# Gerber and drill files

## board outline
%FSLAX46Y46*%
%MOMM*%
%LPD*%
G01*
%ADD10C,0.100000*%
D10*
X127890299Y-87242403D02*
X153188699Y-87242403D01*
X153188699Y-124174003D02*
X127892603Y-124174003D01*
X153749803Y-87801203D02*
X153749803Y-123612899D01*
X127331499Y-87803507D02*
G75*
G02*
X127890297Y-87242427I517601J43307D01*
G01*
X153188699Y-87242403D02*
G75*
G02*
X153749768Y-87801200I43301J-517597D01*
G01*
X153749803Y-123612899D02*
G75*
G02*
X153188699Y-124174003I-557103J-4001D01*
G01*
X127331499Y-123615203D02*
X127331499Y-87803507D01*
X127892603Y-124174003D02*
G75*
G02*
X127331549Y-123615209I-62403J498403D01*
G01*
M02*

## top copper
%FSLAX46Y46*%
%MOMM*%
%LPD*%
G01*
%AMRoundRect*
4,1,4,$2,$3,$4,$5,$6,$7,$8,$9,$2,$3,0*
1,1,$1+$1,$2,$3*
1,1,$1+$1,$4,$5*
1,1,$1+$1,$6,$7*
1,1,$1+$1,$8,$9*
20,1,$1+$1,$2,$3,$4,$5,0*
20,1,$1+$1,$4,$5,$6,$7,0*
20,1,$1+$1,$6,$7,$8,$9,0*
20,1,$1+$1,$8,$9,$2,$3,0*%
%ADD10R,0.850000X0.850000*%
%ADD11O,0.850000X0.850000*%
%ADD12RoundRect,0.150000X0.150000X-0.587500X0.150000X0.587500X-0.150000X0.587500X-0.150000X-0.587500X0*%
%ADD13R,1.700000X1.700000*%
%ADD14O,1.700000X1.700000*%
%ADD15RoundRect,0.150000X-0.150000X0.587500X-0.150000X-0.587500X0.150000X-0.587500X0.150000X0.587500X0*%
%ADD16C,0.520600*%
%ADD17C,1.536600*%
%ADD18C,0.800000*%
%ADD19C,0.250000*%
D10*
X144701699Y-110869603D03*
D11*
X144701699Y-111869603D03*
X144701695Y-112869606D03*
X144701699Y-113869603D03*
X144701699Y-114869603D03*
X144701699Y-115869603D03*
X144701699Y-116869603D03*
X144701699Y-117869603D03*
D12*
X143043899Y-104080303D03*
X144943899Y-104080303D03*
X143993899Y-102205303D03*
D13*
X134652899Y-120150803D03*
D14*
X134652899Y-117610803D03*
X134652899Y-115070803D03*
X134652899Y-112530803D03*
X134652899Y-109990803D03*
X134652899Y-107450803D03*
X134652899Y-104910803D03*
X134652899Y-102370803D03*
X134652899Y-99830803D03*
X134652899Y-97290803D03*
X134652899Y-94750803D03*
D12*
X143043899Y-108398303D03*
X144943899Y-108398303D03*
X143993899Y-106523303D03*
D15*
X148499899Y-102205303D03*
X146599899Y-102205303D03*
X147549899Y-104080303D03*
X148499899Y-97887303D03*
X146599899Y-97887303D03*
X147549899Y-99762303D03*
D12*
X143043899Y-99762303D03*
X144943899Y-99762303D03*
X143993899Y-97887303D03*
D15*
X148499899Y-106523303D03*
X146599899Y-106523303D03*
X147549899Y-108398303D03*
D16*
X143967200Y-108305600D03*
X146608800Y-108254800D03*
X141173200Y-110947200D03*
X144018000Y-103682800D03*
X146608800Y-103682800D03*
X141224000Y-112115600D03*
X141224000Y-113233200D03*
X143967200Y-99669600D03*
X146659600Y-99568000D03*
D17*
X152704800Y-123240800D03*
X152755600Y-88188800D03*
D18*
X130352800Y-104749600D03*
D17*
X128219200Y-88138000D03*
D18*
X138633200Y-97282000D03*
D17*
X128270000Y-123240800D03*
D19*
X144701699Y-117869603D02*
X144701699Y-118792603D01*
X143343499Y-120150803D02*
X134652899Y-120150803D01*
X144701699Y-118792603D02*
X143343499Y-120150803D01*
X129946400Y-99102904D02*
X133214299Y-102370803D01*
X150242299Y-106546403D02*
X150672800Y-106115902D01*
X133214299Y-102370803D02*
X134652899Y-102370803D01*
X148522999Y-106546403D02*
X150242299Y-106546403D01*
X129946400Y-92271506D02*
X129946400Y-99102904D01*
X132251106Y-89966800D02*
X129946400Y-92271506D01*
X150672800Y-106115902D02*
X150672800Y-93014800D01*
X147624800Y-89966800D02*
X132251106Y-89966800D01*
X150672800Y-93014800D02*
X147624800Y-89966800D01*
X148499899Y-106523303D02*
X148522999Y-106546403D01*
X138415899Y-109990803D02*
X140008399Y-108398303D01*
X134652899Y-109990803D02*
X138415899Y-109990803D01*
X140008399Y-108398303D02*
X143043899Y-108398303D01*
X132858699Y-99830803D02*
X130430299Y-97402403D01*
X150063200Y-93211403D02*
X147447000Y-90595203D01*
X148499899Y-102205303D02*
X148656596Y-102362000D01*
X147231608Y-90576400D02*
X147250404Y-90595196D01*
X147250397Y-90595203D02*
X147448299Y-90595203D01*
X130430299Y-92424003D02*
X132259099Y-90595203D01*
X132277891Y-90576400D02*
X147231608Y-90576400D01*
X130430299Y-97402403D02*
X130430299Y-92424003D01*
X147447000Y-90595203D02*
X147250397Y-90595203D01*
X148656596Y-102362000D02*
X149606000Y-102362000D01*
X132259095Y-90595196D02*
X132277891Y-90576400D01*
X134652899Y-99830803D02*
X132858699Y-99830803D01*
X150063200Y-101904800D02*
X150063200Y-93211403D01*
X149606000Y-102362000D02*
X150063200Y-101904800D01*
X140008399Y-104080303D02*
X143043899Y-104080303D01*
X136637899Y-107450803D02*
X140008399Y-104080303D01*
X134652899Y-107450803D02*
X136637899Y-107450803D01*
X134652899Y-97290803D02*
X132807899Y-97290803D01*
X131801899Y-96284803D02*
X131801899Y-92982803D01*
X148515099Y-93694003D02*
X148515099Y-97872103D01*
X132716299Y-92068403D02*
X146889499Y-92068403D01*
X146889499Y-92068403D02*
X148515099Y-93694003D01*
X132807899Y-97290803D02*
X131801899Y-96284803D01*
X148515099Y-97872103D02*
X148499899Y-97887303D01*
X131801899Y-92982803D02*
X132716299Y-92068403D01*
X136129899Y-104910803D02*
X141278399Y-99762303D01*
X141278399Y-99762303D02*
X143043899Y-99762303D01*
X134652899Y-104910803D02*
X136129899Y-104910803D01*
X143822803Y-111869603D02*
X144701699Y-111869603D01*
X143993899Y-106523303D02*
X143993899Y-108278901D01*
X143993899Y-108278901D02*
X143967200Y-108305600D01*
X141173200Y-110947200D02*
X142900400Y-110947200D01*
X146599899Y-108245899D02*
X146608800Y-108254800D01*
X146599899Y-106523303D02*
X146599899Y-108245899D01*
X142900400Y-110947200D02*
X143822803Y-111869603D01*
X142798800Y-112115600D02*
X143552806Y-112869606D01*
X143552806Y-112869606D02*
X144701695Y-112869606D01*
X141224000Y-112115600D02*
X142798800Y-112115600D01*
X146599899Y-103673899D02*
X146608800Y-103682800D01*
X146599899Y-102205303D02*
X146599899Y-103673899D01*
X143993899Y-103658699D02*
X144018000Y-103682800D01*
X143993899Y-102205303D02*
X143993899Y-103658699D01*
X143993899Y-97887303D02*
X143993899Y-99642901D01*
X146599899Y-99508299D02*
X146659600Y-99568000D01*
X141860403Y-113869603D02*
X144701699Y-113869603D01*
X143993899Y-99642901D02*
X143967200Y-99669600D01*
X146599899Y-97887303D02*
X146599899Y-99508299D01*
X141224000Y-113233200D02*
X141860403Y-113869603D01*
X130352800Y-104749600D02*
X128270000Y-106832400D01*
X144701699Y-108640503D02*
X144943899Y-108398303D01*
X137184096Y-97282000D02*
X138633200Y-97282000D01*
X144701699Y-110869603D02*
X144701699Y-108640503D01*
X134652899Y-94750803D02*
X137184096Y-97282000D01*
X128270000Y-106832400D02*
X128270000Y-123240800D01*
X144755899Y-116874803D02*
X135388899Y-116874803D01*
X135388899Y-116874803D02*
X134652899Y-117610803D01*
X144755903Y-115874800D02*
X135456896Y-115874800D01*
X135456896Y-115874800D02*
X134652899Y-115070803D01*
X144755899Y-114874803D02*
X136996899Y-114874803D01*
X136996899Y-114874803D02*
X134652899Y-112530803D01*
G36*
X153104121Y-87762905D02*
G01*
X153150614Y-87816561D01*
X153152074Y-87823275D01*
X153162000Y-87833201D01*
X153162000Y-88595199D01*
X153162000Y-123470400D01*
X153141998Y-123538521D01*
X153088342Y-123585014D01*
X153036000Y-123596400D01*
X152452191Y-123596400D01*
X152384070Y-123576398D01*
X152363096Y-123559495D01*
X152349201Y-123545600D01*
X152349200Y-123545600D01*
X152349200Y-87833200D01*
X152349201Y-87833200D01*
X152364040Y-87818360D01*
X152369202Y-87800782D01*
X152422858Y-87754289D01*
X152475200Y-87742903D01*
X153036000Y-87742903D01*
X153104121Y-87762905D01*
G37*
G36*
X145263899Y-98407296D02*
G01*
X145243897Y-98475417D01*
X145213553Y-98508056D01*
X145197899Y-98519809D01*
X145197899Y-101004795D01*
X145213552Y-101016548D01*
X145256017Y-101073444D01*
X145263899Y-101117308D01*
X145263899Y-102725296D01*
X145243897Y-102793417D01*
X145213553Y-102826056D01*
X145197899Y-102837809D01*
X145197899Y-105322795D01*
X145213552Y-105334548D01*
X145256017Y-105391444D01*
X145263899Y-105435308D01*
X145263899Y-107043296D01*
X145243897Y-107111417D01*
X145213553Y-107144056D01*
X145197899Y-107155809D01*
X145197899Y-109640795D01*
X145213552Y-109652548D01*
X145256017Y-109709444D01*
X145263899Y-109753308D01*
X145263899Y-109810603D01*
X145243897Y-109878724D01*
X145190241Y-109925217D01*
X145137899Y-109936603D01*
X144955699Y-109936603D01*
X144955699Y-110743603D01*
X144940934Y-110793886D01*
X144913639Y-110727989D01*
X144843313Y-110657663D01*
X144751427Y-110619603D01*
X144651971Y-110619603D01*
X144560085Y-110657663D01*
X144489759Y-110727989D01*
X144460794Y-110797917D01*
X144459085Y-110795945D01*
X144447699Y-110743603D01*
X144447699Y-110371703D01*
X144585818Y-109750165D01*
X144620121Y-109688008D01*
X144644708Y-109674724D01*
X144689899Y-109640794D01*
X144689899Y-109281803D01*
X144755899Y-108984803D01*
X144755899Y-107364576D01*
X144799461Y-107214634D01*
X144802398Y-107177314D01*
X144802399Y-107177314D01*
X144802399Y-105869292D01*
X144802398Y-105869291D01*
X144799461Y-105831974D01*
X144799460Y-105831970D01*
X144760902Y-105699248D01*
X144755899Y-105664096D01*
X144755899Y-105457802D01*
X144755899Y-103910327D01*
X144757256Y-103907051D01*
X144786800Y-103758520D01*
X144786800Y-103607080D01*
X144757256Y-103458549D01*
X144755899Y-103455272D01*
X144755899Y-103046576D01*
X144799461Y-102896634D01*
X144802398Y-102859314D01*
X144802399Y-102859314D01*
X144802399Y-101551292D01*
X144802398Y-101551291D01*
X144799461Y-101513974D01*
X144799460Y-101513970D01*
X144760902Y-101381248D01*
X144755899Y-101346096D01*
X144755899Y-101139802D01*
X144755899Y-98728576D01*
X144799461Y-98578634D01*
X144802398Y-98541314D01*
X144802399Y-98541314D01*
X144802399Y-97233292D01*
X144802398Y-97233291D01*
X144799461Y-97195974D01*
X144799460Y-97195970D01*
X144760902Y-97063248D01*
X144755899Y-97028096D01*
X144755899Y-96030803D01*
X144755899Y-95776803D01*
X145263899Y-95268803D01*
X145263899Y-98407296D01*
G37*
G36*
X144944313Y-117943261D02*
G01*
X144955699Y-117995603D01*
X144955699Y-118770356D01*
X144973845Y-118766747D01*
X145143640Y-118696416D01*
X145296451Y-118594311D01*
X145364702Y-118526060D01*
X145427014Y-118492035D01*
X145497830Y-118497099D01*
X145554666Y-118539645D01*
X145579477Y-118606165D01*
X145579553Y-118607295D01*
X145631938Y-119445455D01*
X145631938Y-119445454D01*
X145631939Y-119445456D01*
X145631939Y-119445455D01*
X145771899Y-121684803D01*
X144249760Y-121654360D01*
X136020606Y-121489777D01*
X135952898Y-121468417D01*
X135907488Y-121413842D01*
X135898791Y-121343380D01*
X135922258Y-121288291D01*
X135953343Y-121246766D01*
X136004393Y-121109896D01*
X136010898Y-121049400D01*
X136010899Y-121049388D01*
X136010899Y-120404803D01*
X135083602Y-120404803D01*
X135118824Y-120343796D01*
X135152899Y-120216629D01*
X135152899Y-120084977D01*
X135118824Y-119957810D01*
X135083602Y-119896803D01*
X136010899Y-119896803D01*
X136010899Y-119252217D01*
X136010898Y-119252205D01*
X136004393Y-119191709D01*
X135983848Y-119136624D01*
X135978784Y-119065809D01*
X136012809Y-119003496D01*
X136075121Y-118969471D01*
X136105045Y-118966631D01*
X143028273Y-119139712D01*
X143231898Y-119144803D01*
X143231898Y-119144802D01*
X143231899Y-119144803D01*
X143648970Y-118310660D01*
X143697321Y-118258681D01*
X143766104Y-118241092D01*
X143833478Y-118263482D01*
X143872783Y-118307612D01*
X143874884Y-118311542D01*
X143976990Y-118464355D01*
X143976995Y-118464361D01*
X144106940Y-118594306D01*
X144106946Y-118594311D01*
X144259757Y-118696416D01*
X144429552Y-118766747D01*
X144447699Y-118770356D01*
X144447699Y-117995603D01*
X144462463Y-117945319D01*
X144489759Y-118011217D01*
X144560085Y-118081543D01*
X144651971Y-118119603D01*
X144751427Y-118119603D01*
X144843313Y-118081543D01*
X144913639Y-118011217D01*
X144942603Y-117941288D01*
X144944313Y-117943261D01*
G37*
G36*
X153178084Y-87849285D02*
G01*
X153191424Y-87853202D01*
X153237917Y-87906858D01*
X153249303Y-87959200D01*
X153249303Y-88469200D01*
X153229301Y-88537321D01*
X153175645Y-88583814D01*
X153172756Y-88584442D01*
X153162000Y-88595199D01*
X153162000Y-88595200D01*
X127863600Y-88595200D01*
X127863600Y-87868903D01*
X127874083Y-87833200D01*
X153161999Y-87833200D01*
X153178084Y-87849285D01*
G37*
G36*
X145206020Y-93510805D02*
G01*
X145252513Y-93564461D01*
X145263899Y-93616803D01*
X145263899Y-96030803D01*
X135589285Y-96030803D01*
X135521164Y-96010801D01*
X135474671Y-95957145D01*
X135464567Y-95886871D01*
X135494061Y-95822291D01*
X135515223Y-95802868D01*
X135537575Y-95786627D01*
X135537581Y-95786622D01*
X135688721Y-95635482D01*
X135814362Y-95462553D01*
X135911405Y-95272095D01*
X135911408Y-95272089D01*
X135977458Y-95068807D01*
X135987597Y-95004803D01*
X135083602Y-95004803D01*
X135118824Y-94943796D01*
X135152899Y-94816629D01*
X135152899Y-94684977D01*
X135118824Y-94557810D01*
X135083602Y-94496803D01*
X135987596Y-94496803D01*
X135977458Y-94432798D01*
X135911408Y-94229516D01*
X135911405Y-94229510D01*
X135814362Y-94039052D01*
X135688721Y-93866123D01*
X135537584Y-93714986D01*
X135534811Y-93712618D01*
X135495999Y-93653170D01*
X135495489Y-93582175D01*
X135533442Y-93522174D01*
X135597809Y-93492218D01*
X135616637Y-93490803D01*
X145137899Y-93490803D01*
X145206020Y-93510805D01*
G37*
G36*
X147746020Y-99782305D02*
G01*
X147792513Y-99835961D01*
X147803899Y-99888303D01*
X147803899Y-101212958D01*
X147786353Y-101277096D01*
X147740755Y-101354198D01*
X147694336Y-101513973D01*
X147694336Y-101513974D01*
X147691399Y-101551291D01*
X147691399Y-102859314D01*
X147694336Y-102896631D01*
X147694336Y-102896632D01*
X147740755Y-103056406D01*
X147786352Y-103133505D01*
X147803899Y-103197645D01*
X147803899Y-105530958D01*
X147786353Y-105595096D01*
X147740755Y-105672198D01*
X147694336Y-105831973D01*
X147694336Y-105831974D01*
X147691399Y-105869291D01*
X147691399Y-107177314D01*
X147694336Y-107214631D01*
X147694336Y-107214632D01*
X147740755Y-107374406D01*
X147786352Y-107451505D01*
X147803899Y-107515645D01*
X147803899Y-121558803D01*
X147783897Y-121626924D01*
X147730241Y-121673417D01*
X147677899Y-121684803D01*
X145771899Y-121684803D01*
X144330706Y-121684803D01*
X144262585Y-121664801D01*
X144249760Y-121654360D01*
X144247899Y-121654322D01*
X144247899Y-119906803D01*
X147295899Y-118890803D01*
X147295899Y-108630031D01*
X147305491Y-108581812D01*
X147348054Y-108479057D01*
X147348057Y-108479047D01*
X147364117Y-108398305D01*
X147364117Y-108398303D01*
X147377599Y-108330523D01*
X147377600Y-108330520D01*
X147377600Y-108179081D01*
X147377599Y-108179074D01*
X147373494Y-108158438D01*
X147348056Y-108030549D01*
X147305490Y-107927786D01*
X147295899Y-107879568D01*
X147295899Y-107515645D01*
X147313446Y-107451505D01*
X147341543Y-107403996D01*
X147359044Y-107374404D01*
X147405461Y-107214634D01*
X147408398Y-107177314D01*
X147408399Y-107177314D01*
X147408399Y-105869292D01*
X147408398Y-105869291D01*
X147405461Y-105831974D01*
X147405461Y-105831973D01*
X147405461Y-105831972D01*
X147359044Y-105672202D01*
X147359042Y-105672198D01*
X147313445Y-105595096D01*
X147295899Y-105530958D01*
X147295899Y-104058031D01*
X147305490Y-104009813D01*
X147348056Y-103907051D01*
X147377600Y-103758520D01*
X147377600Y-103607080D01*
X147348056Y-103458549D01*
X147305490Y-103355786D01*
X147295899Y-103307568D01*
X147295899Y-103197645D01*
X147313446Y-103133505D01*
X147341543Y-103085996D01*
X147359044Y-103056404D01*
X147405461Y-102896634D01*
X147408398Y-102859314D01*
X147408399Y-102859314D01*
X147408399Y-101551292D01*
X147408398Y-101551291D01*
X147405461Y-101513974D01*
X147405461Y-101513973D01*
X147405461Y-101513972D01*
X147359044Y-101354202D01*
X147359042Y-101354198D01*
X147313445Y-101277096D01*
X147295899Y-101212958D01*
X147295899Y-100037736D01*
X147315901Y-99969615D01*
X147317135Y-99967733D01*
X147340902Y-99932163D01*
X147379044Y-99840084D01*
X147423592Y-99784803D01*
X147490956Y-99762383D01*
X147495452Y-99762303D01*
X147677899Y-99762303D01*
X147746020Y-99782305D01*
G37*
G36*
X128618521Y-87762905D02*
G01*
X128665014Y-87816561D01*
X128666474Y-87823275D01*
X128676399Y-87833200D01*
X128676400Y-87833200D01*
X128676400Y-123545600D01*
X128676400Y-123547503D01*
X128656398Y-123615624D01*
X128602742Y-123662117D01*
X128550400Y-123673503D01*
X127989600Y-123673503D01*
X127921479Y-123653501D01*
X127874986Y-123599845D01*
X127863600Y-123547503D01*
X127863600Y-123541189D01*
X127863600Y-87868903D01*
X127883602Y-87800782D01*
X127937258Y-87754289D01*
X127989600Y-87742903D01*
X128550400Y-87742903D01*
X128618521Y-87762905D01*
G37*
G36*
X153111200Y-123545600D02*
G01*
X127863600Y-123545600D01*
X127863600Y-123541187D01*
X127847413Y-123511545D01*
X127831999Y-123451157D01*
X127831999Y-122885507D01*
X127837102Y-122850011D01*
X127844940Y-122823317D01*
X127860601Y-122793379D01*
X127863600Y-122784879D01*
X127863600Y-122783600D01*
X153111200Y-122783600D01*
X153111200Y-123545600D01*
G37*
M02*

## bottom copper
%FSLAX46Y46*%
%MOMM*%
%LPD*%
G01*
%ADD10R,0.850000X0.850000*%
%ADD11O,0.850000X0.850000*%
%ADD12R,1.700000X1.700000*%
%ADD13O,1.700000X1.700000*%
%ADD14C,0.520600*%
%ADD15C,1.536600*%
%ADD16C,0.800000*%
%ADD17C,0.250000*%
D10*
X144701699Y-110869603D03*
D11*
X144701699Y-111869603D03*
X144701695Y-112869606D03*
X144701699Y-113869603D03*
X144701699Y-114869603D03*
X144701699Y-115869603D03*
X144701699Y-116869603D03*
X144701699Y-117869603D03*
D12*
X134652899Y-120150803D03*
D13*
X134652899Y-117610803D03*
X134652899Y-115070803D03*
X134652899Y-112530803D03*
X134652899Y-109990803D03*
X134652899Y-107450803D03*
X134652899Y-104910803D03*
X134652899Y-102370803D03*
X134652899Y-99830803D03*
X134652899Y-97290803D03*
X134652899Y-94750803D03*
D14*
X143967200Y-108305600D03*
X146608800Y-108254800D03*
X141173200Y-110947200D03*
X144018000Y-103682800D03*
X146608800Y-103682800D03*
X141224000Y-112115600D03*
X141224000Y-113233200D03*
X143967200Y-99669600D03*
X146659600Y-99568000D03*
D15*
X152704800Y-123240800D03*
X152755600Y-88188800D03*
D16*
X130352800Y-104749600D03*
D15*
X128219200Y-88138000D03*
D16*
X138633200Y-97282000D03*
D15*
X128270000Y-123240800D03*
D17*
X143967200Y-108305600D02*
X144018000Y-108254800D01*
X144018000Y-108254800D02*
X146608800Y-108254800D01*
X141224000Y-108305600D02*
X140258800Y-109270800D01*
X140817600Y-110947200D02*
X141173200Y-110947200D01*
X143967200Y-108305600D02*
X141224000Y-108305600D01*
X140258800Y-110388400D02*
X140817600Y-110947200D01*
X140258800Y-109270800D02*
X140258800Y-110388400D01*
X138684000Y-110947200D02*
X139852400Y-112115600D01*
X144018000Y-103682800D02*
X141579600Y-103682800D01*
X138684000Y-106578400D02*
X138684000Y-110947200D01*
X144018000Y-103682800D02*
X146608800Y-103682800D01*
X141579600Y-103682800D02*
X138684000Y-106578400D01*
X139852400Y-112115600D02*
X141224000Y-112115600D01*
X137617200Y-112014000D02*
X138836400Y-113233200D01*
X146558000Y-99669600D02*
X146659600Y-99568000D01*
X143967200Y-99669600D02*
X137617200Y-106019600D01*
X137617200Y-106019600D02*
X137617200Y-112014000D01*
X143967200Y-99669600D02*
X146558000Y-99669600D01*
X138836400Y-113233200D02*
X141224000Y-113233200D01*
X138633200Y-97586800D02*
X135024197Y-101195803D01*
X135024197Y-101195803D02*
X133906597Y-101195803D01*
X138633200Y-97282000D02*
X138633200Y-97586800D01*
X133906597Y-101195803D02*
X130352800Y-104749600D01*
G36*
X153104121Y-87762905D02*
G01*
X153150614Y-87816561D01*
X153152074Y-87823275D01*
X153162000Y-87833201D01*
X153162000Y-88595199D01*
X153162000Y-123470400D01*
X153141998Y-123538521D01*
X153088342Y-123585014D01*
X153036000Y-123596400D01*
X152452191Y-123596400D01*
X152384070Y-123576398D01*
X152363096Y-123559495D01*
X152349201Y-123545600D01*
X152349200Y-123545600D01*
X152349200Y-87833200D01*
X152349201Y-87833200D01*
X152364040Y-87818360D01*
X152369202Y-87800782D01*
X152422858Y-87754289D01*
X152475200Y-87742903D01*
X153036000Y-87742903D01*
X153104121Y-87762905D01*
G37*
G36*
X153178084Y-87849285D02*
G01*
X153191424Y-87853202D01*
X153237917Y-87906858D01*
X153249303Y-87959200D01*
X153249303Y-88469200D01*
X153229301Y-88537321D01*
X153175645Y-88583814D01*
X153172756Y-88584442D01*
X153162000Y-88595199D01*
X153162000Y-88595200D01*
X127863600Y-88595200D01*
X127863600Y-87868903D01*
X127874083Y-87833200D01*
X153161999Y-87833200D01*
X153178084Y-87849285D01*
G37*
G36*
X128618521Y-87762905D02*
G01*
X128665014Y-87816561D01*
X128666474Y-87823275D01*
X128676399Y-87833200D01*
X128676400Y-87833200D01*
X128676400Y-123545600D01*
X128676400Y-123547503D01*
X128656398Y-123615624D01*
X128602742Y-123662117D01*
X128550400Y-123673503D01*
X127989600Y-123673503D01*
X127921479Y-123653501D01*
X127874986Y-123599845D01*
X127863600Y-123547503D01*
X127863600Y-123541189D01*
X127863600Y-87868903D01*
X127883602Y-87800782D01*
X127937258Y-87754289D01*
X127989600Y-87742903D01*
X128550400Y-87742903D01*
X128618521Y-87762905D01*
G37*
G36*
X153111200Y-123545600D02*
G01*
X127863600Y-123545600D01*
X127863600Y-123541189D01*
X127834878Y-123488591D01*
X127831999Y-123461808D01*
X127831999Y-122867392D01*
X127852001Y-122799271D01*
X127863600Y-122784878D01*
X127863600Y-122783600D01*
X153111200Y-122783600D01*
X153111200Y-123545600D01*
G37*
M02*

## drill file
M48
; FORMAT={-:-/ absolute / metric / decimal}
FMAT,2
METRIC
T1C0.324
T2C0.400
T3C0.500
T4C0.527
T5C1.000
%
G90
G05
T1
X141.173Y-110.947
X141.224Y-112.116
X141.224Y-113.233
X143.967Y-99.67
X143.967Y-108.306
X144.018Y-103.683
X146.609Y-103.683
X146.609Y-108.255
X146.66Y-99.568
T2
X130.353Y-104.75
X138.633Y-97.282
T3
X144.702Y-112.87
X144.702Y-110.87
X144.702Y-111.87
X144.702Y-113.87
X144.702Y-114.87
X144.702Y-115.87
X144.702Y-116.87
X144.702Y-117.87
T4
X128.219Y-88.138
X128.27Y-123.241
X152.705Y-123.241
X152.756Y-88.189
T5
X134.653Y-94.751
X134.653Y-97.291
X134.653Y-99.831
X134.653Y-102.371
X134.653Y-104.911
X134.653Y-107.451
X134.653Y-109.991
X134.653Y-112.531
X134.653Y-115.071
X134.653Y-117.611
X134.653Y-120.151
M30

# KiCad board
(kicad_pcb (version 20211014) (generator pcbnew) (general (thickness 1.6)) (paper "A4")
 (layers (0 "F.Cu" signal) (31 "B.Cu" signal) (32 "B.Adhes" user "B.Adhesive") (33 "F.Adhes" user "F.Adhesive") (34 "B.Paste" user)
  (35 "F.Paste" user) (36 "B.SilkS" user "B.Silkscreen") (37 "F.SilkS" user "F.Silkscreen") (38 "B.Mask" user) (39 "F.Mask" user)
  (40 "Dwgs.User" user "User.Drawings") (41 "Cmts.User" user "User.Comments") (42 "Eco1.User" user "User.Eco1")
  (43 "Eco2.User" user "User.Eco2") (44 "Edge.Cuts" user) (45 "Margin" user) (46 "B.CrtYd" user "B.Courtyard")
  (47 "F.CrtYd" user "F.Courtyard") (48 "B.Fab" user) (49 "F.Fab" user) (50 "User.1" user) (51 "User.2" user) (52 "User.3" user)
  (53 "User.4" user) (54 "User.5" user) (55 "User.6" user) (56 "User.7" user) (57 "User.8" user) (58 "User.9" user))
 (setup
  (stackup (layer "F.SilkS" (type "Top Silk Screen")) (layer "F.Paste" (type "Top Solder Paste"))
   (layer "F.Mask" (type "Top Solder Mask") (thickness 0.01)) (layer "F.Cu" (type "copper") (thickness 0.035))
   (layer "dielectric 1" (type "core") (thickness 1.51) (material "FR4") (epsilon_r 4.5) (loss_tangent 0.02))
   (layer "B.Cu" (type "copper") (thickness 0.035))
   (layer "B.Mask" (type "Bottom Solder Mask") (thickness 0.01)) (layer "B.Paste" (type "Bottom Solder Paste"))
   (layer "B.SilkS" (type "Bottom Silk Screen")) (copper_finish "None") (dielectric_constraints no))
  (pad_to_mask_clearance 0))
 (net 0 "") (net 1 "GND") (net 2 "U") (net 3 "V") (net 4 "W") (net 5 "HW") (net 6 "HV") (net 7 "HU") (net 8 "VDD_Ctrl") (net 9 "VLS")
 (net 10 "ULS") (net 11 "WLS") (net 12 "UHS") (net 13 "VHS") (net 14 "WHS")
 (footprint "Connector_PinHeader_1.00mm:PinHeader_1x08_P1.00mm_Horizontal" (layer "F.Cu") (at 144.701699 110.869603)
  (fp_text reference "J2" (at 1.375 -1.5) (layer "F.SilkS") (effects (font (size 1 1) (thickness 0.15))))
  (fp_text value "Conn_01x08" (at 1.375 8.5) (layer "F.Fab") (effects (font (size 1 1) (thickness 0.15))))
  (pad "1" thru_hole rect (at 0 0) (size 0.85 0.85) (drill 0.5) (layers *.Cu *.Mask) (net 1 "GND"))
  (pad "2" thru_hole oval (at 0 1) (size 0.85 0.85) (drill 0.5) (layers *.Cu *.Mask) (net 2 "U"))
  (pad "3" thru_hole oval (at -0.000004 2.000003) (size 0.85 0.85) (drill 0.5) (layers *.Cu *.Mask) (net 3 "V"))
  (pad "4" thru_hole oval (at 0 3) (size 0.85 0.85) (drill 0.5) (layers *.Cu *.Mask) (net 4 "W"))
  (pad "5" thru_hole oval (at 0 4) (size 0.85 0.85) (drill 0.5) (layers *.Cu *.Mask) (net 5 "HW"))
  (pad "6" thru_hole oval (at 0 5) (size 0.85 0.85) (drill 0.5) (layers *.Cu *.Mask) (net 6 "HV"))
  (pad "7" thru_hole oval (at 0 6) (size 0.85 0.85) (drill 0.5) (layers *.Cu *.Mask) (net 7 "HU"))
  (pad "8" thru_hole oval (at 0 7) (size 0.85 0.85) (drill 0.5) (layers *.Cu *.Mask) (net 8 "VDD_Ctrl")))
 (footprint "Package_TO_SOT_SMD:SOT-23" (layer "F.Cu") (at 143.993899 103.142803 90)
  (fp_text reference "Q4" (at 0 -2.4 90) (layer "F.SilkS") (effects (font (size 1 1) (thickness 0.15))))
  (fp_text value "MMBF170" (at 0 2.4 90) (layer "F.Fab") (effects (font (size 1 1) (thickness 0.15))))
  (pad "1" smd roundrect (at -0.9375 -0.95 90) (size 1.475 0.6) (layers "F.Cu" "F.Paste" "F.Mask") (roundrect_rratio 0.25) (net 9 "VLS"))
  (pad "2" smd roundrect (at -0.9375 0.95 90) (size 1.475 0.6) (layers "F.Cu" "F.Paste" "F.Mask") (roundrect_rratio 0.25) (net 1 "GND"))
  (pad "3" smd roundrect (at 0.9375 0 90) (size 1.475 0.6) (layers "F.Cu" "F.Paste" "F.Mask") (roundrect_rratio 0.25) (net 3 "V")))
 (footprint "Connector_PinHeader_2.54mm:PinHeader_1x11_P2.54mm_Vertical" (layer "F.Cu") (at 134.652899 120.150803 180)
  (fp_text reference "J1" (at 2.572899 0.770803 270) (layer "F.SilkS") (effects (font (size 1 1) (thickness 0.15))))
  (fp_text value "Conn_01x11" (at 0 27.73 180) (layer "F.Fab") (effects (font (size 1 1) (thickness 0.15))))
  (pad "1" thru_hole rect (at 0 0 180) (size 1.7 1.7) (drill 1) (layers *.Cu *.Mask) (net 8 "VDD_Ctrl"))
  (pad "2" thru_hole oval (at 0 2.54 180) (size 1.7 1.7) (drill 1) (layers *.Cu *.Mask) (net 7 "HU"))
  (pad "3" thru_hole oval (at 0 5.08 180) (size 1.7 1.7) (drill 1) (layers *.Cu *.Mask) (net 6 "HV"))
  (pad "4" thru_hole oval (at 0 7.62 180) (size 1.7 1.7) (drill 1) (layers *.Cu *.Mask) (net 5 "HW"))
  (pad "5" thru_hole oval (at 0 10.16 180) (size 1.7 1.7) (drill 1) (layers *.Cu *.Mask) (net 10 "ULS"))
  (pad "6" thru_hole oval (at 0 12.7 180) (size 1.7 1.7) (drill 1) (layers *.Cu *.Mask) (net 9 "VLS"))
  (pad "7" thru_hole oval (at 0 15.24 180) (size 1.7 1.7) (drill 1) (layers *.Cu *.Mask) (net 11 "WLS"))
  (pad "8" thru_hole oval (at 0 17.78 180) (size 1.7 1.7) (drill 1) (layers *.Cu *.Mask) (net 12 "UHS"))
  (pad "9" thru_hole oval (at 0 20.32 180) (size 1.7 1.7) (drill 1) (layers *.Cu *.Mask) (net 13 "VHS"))
  (pad "10" thru_hole oval (at 0 22.86 180) (size 1.7 1.7) (drill 1) (layers *.Cu *.Mask) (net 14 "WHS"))
  (pad "11" thru_hole oval (at 0 25.4 180) (size 1.7 1.7) (drill 1) (layers *.Cu *.Mask) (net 1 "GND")))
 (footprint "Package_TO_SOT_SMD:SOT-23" (layer "F.Cu") (at 143.993899 107.460803 90)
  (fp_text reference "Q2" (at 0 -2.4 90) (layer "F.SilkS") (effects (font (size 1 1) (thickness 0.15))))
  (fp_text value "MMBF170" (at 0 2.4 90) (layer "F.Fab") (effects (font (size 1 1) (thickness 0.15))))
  (pad "1" smd roundrect (at -0.9375 -0.95 90) (size 1.475 0.6) (layers "F.Cu" "F.Paste" "F.Mask") (roundrect_rratio 0.25) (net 10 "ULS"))
  (pad "2" smd roundrect (at -0.9375 0.95 90) (size 1.475 0.6) (layers "F.Cu" "F.Paste" "F.Mask") (roundrect_rratio 0.25) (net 1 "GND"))
  (pad "3" smd roundrect (at 0.9375 0 90) (size 1.475 0.6) (layers "F.Cu" "F.Paste" "F.Mask") (roundrect_rratio 0.25) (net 2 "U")))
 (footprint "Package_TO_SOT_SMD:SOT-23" (layer "F.Cu") (at 147.549899 103.142803 -90)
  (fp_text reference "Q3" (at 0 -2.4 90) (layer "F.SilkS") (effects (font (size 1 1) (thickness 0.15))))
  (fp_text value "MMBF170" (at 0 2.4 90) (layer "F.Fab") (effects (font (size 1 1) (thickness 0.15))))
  (pad "1" smd roundrect (at -0.9375 -0.95 270) (size 1.475 0.6) (layers "F.Cu" "F.Paste" "F.Mask") (roundrect_rratio 0.25) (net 13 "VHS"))
  (pad "2" smd roundrect (at -0.9375 0.95 270) (size 1.475 0.6) (layers "F.Cu" "F.Paste" "F.Mask") (roundrect_rratio 0.25) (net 3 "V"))
  (pad "3" smd roundrect (at 0.9375 0 270) (size 1.475 0.6) (layers "F.Cu" "F.Paste" "F.Mask") (roundrect_rratio 0.25) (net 8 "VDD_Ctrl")))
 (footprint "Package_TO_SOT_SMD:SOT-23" (layer "F.Cu") (at 147.549899 98.824803 -90)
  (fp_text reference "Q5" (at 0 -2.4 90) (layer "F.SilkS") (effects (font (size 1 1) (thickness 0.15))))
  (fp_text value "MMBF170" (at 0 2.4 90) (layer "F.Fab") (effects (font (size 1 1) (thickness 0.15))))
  (pad "1" smd roundrect (at -0.9375 -0.95 270) (size 1.475 0.6) (layers "F.Cu" "F.Paste" "F.Mask") (roundrect_rratio 0.25) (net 14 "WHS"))
  (pad "2" smd roundrect (at -0.9375 0.95 270) (size 1.475 0.6) (layers "F.Cu" "F.Paste" "F.Mask") (roundrect_rratio 0.25) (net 4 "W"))
  (pad "3" smd roundrect (at 0.9375 0 270) (size 1.475 0.6) (layers "F.Cu" "F.Paste" "F.Mask") (roundrect_rratio 0.25) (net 8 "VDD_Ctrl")))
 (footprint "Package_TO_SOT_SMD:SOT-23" (layer "F.Cu") (at 143.993899 98.824803 90)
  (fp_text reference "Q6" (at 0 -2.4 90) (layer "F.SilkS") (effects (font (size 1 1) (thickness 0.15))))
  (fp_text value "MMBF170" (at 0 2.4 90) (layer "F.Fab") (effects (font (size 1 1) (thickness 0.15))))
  (pad "1" smd roundrect (at -0.9375 -0.95 90) (size 1.475 0.6) (layers "F.Cu" "F.Paste" "F.Mask") (roundrect_rratio 0.25) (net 11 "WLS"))
  (pad "2" smd roundrect (at -0.9375 0.95 90) (size 1.475 0.6) (layers "F.Cu" "F.Paste" "F.Mask") (roundrect_rratio 0.25) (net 1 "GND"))
  (pad "3" smd roundrect (at 0.9375 0 90) (size 1.475 0.6) (layers "F.Cu" "F.Paste" "F.Mask") (roundrect_rratio 0.25) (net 4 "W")))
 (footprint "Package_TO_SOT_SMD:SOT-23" (layer "F.Cu") (at 147.549899 107.460803 -90)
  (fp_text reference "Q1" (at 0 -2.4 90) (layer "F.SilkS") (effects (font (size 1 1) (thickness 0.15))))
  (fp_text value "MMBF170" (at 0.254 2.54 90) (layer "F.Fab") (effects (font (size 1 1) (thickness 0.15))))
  (pad "1" smd roundrect (at -0.9375 -0.95 270) (size 1.475 0.6) (layers "F.Cu" "F.Paste" "F.Mask") (roundrect_rratio 0.25) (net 12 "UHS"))
  (pad "2" smd roundrect (at -0.9375 0.95 270) (size 1.475 0.6) (layers "F.Cu" "F.Paste" "F.Mask") (roundrect_rratio 0.25) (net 2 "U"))
  (pad "3" smd roundrect (at 0.9375 0 270) (size 1.475 0.6) (layers "F.Cu" "F.Paste" "F.Mask") (roundrect_rratio 0.25) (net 8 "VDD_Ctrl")))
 (gr_line (start 127.890299 87.242403) (end 153.188699 87.242403) (layer "Edge.Cuts") (width 0.1))
 (gr_line (start 153.188699 124.174003) (end 127.892603 124.174003) (layer "Edge.Cuts") (width 0.1))
 (gr_line (start 153.749803 87.801203) (end 153.749803 123.612899) (layer "Edge.Cuts") (width 0.1))
 (gr_arc (start 127.331499 87.803507) (mid 127.481074 87.393663) (end 127.890299 87.242403) (layer "Edge.Cuts") (width 0.1))
 (gr_arc (start 153.188699 87.242403) (mid 153.598538 87.391982) (end 153.749803 87.801203) (layer "Edge.Cuts") (width 0.1))
 (gr_arc (start 153.749803 123.612899) (mid 153.586636 124.010836) (end 153.188699 124.174003) (layer "Edge.Cuts") (width 0.1))
 (gr_line (start 127.331499 123.615203) (end 127.331499 87.803507) (layer "Edge.Cuts") (width 0.1))
 (gr_arc (start 127.892603 124.174003) (mid 127.475721 124.031493) (end 127.331499 123.615203) (layer "Edge.Cuts") (width 0.1))
 (segment (start 144.701699 117.869603) (end 144.701699 118.792603) (width 0.25) (layer "F.Cu") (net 8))
 (segment (start 143.343499 120.150803) (end 134.652899 120.150803) (width 0.25) (layer "F.Cu") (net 8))
 (segment (start 144.701699 118.792603) (end 143.343499 120.150803) (width 0.25) (layer "F.Cu") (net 8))
 (segment (start 129.9464 99.102904) (end 133.214299 102.370803) (width 0.25) (layer "F.Cu") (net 12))
 (segment (start 150.242299 106.546403) (end 150.6728 106.115902) (width 0.25) (layer "F.Cu") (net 12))
 (segment (start 133.214299 102.370803) (end 134.652899 102.370803) (width 0.25) (layer "F.Cu") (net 12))
 (segment (start 148.522999 106.546403) (end 150.242299 106.546403) (width 0.25) (layer "F.Cu") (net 12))
 (segment (start 129.9464 92.271506) (end 129.9464 99.102904) (width 0.25) (layer "F.Cu") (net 12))
 (segment (start 132.251106 89.9668) (end 129.9464 92.271506) (width 0.25) (layer "F.Cu") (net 12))
 (segment (start 150.6728 106.115902) (end 150.6728 93.0148) (width 0.25) (layer "F.Cu") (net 12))
 (segment (start 147.6248 89.9668) (end 132.251106 89.9668) (width 0.25) (layer "F.Cu") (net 12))
 (segment (start 150.6728 93.0148) (end 147.6248 89.9668) (width 0.25) (layer "F.Cu") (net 12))
 (segment (start 148.499899 106.523303) (end 148.522999 106.546403) (width 0.25) (layer "F.Cu") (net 12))
 (segment (start 138.415899 109.990803) (end 140.008399 108.398303) (width 0.25) (layer "F.Cu") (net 10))
 (segment (start 134.652899 109.990803) (end 138.415899 109.990803) (width 0.25) (layer "F.Cu") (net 10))
 (segment (start 140.008399 108.398303) (end 143.043899 108.398303) (width 0.25) (layer "F.Cu") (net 10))
 (segment (start 132.858699 99.830803) (end 130.430299 97.402403) (width 0.25) (layer "F.Cu") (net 13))
 (segment (start 150.0632 93.211403) (end 147.447 90.595203) (width 0.25) (layer "F.Cu") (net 13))
 (segment (start 148.499899 102.205303) (end 148.656596 102.362) (width 0.25) (layer "F.Cu") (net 13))
 (segment (start 147.231608 90.5764) (end 147.250404 90.595196) (width 0.25) (layer "F.Cu") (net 13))
 (segment (start 147.250397 90.595203) (end 147.448299 90.595203) (width 0.25) (layer "F.Cu") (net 13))
 (segment (start 130.430299 92.424003) (end 132.259099 90.595203) (width 0.25) (layer "F.Cu") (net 13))
 (segment (start 132.277891 90.5764) (end 147.231608 90.5764) (width 0.25) (layer "F.Cu") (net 13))
 (segment (start 130.430299 97.402403) (end 130.430299 92.424003) (width 0.25) (layer "F.Cu") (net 13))
 (segment (start 147.447 90.595203) (end 147.250397 90.595203) (width 0.25) (layer "F.Cu") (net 13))
 (segment (start 148.656596 102.362) (end 149.606 102.362) (width 0.25) (layer "F.Cu") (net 13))
 (segment (start 132.259095 90.595196) (end 132.277891 90.5764) (width 0.25) (layer "F.Cu") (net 13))
 (segment (start 134.652899 99.830803) (end 132.858699 99.830803) (width 0.25) (layer "F.Cu") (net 13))
 (segment (start 150.0632 101.9048) (end 150.0632 93.211403) (width 0.25) (layer "F.Cu") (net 13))
 (segment (start 149.606 102.362) (end 150.0632 101.9048) (width 0.25) (layer "F.Cu") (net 13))
 (segment (start 140.008399 104.080303) (end 143.043899 104.080303) (width 0.25) (layer "F.Cu") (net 9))
 (segment (start 136.637899 107.450803) (end 140.008399 104.080303) (width 0.25) (layer "F.Cu") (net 9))
 (segment (start 134.652899 107.450803) (end 136.637899 107.450803) (width 0.25) (layer "F.Cu") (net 9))
 (segment (start 134.652899 97.290803) (end 132.807899 97.290803) (width 0.25) (layer "F.Cu") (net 14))
 (segment (start 131.801899 96.284803) (end 131.801899 92.982803) (width 0.25) (layer "F.Cu") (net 14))
 (segment (start 148.515099 93.694003) (end 148.515099 97.872103) (width 0.25) (layer "F.Cu") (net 14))
 (segment (start 132.716299 92.068403) (end 146.889499 92.068403) (width 0.25) (layer "F.Cu") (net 14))
 (segment (start 146.889499 92.068403) (end 148.515099 93.694003) (width 0.25) (layer "F.Cu") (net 14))
 (segment (start 132.807899 97.290803) (end 131.801899 96.284803) (width 0.25) (layer "F.Cu") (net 14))
 (segment (start 148.515099 97.872103) (end 148.499899 97.887303) (width 0.25) (layer "F.Cu") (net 14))
 (segment (start 131.801899 92.982803) (end 132.716299 92.068403) (width 0.25) (layer "F.Cu") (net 14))
 (segment (start 136.129899 104.910803) (end 141.278399 99.762303) (width 0.25) (layer "F.Cu") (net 11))
 (segment (start 141.278399 99.762303) (end 143.043899 99.762303) (width 0.25) (layer "F.Cu") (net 11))
 (segment (start 134.652899 104.910803) (end 136.129899 104.910803) (width 0.25) (layer "F.Cu") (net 11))
 (segment (start 143.822803 111.869603) (end 144.701699 111.869603) (width 0.25) (layer "F.Cu") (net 2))
 (segment (start 143.993899 106.523303) (end 143.993899 108.278901) (width 0.25) (layer "F.Cu") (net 2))
 (segment (start 143.993899 108.278901) (end 143.9672 108.3056) (width 0.25) (layer "F.Cu") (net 2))
 (segment (start 141.1732 110.9472) (end 142.9004 110.9472) (width 0.25) (layer "F.Cu") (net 2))
 (segment (start 146.599899 108.245899) (end 146.6088 108.2548) (width 0.25) (layer "F.Cu") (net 2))
 (segment (start 146.599899 106.523303) (end 146.599899 108.245899) (width 0.25) (layer "F.Cu") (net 2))
 (segment (start 142.9004 110.9472) (end 143.822803 111.869603) (width 0.25) (layer "F.Cu") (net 2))
 (via (at 143.9672 108.3056) (size 0.5206) (drill 0.3238) (layers "F.Cu" "B.Cu") (free) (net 2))
 (via (at 146.6088 108.2548) (size 0.5206) (drill 0.3238) (layers "F.Cu" "B.Cu") (free) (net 2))
 (via (at 141.1732 110.9472) (size 0.5206) (drill 0.3238) (layers "F.Cu" "B.Cu") (free) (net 2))
 (segment (start 143.9672 108.3056) (end 144.018 108.2548) (width 0.25) (layer "B.Cu") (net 2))
 (segment (start 144.018 108.2548) (end 146.6088 108.2548) (width 0.25) (layer "B.Cu") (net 2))
 (segment (start 141.224 108.3056) (end 140.2588 109.2708) (width 0.25) (layer "B.Cu") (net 2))
 (segment (start 140.8176 110.9472) (end 141.1732 110.9472) (width 0.25) (layer "B.Cu") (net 2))
 (segment (start 143.9672 108.3056) (end 141.224 108.3056) (width 0.25) (layer "B.Cu") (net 2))
 (segment (start 140.2588 110.3884) (end 140.8176 110.9472) (width 0.25) (layer "B.Cu") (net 2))
 (segment (start 140.2588 109.2708) (end 140.2588 110.3884) (width 0.25) (layer "B.Cu") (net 2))
 (segment (start 142.7988 112.1156) (end 143.552806 112.869606) (width 0.25) (layer "F.Cu") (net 3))
 (segment (start 143.552806 112.869606) (end 144.701695 112.869606) (width 0.25) (layer "F.Cu") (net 3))
 (segment (start 141.224 112.1156) (end 142.7988 112.1156) (width 0.25) (layer "F.Cu") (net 3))
 (segment (start 146.599899 103.673899) (end 146.6088 103.6828) (width 0.25) (layer "F.Cu") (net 3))
 (segment (start 146.599899 102.205303) (end 146.599899 103.673899) (width 0.25) (layer "F.Cu") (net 3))
 (segment (start 143.993899 103.658699) (end 144.018 103.6828) (width 0.25) (layer "F.Cu") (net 3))
 (segment (start 143.993899 102.205303) (end 143.993899 103.658699) (width 0.25) (layer "F.Cu") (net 3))
 (via (at 144.018 103.6828) (size 0.5206) (drill 0.3238) (layers "F.Cu" "B.Cu") (free) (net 3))
 (via (at 146.6088 103.6828) (size 0.5206) (drill 0.3238) (layers "F.Cu" "B.Cu") (free) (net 3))
 (via (at 141.224 112.1156) (size 0.5206) (drill 0.3238) (layers "F.Cu" "B.Cu") (free) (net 3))
 (segment (start 138.684 110.9472) (end 139.8524 112.1156) (width 0.25) (layer "B.Cu") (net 3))
 (segment (start 144.018 103.6828) (end 141.5796 103.6828) (width 0.25) (layer "B.Cu") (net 3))
 (segment (start 138.684 106.5784) (end 138.684 110.9472) (width 0.25) (layer "B.Cu") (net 3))
 (segment (start 144.018 103.6828) (end 146.6088 103.6828) (width 0.25) (layer "B.Cu") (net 3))
 (segment (start 141.5796 103.6828) (end 138.684 106.5784) (width 0.25) (layer "B.Cu") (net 3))
 (segment (start 139.8524 112.1156) (end 141.224 112.1156) (width 0.25) (layer "B.Cu") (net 3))
 (segment (start 143.993899 97.887303) (end 143.993899 99.642901) (width 0.25) (layer "F.Cu") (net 4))
 (segment (start 146.599899 99.508299) (end 146.6596 99.568) (width 0.25) (layer "F.Cu") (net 4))
 (segment (start 141.860403 113.869603) (end 144.701699 113.869603) (width 0.25) (layer "F.Cu") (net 4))
 (segment (start 143.993899 99.642901) (end 143.9672 99.6696) (width 0.25) (layer "F.Cu") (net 4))
 (segment (start 146.599899 97.887303) (end 146.599899 99.508299) (width 0.25) (layer "F.Cu") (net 4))
 (segment (start 141.224 113.2332) (end 141.860403 113.869603) (width 0.25) (layer "F.Cu") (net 4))
 (via (at 141.224 113.2332) (size 0.5206) (drill 0.3238) (layers "F.Cu" "B.Cu") (free) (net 4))
 (via (at 143.9672 99.6696) (size 0.5206) (drill 0.3238) (layers "F.Cu" "B.Cu") (free) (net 4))
 (via (at 146.6596 99.568) (size 0.5206) (drill 0.3238) (layers "F.Cu" "B.Cu") (free) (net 4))
 (segment (start 137.6172 112.014) (end 138.8364 113.2332) (width 0.25) (layer "B.Cu") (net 4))
 (segment (start 146.558 99.6696) (end 146.6596 99.568) (width 0.25) (layer "B.Cu") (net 4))
 (segment (start 143.9672 99.6696) (end 137.6172 106.0196) (width 0.25) (layer "B.Cu") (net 4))
 (segment (start 137.6172 106.0196) (end 137.6172 112.014) (width 0.25) (layer "B.Cu") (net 4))
 (segment (start 143.9672 99.6696) (end 146.558 99.6696) (width 0.25) (layer "B.Cu") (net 4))
 (segment (start 138.8364 113.2332) (end 141.224 113.2332) (width 0.25) (layer "B.Cu") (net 4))
 (segment (start 130.3528 104.7496) (end 128.27 106.8324) (width 0.25) (layer "F.Cu") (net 1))
 (segment (start 144.701699 108.640503) (end 144.943899 108.398303) (width 0.25) (layer "F.Cu") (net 1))
 (segment (start 137.184096 97.282) (end 138.6332 97.282) (width 0.25) (layer "F.Cu") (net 1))
 (segment (start 144.701699 110.869603) (end 144.701699 108.640503) (width 0.25) (layer "F.Cu") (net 1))
 (segment (start 134.652899 94.750803) (end 137.184096 97.282) (width 0.25) (layer "F.Cu") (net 1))
 (segment (start 128.27 106.8324) (end 128.27 123.2408) (width 0.25) (layer "F.Cu") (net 1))
 (via (at 152.7048 123.2408) (size 1.5366) (drill 0.527) (layers "F.Cu" "B.Cu") (free) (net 1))
 (via (at 152.7556 88.1888) (size 1.5366) (drill 0.527) (layers "F.Cu" "B.Cu") (free) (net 1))
 (via (at 130.3528 104.7496) (size 0.8) (drill 0.4) (layers "F.Cu" "B.Cu") (free) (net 1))
 (via (at 128.2192 88.138) (size 1.5366) (drill 0.527) (layers "F.Cu" "B.Cu") (free) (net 1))
 (via (at 138.6332 97.282) (size 0.8) (drill 0.4) (layers "F.Cu" "B.Cu") (free) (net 1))
 (via (at 128.27 123.2408) (size 1.5366) (drill 0.527) (layers "F.Cu" "B.Cu") (free) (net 1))
 (segment (start 138.6332 97.5868) (end 135.024197 101.195803) (width 0.25) (layer "B.Cu") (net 1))
 (segment (start 135.024197 101.195803) (end 133.906597 101.195803) (width 0.25) (layer "B.Cu") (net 1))
 (segment (start 138.6332 97.282) (end 138.6332 97.5868) (width 0.25) (layer "B.Cu") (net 1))
 (segment (start 133.906597 101.195803) (end 130.3528 104.7496) (width 0.25) (layer "B.Cu") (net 1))
 (segment (start 144.755899 116.874803) (end 135.388899 116.874803) (width 0.25) (layer "F.Cu") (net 7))
 (segment (start 135.388899 116.874803) (end 134.652899 117.610803) (width 0.25) (layer "F.Cu") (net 7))
 (segment (start 144.755903 115.8748) (end 135.456896 115.8748) (width 0.25) (layer "F.Cu") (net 6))
 (segment (start 135.456896 115.8748) (end 134.652899 115.070803) (width 0.25) (layer "F.Cu") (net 6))
 (segment (start 144.755899 114.874803) (end 136.996899 114.874803) (width 0.25) (layer "F.Cu") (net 5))
 (segment (start 136.996899 114.874803) (end 134.652899 112.530803) (width 0.25) (layer "F.Cu") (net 5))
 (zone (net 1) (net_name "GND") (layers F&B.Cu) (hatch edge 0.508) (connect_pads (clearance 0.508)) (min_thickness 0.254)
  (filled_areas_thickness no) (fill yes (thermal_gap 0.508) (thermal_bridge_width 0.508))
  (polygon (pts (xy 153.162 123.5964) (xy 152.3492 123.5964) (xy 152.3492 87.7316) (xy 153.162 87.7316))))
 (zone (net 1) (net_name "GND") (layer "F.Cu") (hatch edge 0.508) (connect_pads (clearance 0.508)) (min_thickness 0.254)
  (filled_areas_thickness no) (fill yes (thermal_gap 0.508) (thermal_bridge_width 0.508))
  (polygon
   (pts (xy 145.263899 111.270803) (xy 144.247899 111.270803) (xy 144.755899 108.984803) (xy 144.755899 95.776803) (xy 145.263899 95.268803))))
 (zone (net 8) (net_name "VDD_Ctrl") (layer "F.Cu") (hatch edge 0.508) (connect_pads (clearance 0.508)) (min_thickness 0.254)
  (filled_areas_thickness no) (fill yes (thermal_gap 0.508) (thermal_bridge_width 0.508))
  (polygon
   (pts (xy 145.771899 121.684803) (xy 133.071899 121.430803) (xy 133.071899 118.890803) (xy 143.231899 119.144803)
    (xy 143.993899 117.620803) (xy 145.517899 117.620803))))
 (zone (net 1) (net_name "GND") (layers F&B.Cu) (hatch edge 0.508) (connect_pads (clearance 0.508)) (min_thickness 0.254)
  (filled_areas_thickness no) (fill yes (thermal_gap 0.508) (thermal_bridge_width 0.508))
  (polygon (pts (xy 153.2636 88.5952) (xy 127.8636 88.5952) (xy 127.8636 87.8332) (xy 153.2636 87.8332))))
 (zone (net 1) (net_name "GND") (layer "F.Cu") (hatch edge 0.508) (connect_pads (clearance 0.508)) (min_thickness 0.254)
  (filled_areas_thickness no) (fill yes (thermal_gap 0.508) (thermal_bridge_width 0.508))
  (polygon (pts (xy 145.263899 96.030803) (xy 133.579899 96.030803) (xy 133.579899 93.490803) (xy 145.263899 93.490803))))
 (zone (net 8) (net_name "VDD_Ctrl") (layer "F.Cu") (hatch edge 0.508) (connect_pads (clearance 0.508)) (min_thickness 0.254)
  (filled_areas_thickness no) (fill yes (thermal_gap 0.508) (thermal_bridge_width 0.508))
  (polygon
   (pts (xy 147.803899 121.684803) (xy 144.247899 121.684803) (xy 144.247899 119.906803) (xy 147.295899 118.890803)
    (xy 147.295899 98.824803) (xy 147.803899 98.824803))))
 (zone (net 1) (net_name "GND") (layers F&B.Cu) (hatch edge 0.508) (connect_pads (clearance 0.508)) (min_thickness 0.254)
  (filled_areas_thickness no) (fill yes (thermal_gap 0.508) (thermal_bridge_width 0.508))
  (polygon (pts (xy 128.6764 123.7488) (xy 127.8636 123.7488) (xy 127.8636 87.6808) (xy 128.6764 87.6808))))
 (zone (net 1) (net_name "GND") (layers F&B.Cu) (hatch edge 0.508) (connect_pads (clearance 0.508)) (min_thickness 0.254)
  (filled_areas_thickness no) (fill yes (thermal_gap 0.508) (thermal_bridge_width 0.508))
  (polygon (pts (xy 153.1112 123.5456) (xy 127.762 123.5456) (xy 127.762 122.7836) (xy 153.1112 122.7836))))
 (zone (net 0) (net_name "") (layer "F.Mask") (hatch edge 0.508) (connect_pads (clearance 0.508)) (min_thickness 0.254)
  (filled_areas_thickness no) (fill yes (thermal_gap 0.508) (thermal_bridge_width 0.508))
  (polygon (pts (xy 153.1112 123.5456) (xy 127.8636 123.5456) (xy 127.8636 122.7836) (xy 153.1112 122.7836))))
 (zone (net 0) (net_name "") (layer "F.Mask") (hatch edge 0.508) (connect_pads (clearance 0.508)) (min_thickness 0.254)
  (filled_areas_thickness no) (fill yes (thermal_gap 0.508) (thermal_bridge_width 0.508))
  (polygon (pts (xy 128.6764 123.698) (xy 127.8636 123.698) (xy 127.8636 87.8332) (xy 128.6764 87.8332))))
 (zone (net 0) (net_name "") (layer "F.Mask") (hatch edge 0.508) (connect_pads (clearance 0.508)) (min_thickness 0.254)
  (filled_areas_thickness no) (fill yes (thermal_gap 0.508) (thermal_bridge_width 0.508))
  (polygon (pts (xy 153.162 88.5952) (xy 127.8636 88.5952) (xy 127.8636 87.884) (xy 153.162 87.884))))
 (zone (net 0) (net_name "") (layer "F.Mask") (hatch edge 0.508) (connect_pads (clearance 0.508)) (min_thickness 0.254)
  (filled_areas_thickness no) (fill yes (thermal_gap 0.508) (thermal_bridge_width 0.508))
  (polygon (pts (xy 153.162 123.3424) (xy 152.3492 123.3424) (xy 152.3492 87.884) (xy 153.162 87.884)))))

